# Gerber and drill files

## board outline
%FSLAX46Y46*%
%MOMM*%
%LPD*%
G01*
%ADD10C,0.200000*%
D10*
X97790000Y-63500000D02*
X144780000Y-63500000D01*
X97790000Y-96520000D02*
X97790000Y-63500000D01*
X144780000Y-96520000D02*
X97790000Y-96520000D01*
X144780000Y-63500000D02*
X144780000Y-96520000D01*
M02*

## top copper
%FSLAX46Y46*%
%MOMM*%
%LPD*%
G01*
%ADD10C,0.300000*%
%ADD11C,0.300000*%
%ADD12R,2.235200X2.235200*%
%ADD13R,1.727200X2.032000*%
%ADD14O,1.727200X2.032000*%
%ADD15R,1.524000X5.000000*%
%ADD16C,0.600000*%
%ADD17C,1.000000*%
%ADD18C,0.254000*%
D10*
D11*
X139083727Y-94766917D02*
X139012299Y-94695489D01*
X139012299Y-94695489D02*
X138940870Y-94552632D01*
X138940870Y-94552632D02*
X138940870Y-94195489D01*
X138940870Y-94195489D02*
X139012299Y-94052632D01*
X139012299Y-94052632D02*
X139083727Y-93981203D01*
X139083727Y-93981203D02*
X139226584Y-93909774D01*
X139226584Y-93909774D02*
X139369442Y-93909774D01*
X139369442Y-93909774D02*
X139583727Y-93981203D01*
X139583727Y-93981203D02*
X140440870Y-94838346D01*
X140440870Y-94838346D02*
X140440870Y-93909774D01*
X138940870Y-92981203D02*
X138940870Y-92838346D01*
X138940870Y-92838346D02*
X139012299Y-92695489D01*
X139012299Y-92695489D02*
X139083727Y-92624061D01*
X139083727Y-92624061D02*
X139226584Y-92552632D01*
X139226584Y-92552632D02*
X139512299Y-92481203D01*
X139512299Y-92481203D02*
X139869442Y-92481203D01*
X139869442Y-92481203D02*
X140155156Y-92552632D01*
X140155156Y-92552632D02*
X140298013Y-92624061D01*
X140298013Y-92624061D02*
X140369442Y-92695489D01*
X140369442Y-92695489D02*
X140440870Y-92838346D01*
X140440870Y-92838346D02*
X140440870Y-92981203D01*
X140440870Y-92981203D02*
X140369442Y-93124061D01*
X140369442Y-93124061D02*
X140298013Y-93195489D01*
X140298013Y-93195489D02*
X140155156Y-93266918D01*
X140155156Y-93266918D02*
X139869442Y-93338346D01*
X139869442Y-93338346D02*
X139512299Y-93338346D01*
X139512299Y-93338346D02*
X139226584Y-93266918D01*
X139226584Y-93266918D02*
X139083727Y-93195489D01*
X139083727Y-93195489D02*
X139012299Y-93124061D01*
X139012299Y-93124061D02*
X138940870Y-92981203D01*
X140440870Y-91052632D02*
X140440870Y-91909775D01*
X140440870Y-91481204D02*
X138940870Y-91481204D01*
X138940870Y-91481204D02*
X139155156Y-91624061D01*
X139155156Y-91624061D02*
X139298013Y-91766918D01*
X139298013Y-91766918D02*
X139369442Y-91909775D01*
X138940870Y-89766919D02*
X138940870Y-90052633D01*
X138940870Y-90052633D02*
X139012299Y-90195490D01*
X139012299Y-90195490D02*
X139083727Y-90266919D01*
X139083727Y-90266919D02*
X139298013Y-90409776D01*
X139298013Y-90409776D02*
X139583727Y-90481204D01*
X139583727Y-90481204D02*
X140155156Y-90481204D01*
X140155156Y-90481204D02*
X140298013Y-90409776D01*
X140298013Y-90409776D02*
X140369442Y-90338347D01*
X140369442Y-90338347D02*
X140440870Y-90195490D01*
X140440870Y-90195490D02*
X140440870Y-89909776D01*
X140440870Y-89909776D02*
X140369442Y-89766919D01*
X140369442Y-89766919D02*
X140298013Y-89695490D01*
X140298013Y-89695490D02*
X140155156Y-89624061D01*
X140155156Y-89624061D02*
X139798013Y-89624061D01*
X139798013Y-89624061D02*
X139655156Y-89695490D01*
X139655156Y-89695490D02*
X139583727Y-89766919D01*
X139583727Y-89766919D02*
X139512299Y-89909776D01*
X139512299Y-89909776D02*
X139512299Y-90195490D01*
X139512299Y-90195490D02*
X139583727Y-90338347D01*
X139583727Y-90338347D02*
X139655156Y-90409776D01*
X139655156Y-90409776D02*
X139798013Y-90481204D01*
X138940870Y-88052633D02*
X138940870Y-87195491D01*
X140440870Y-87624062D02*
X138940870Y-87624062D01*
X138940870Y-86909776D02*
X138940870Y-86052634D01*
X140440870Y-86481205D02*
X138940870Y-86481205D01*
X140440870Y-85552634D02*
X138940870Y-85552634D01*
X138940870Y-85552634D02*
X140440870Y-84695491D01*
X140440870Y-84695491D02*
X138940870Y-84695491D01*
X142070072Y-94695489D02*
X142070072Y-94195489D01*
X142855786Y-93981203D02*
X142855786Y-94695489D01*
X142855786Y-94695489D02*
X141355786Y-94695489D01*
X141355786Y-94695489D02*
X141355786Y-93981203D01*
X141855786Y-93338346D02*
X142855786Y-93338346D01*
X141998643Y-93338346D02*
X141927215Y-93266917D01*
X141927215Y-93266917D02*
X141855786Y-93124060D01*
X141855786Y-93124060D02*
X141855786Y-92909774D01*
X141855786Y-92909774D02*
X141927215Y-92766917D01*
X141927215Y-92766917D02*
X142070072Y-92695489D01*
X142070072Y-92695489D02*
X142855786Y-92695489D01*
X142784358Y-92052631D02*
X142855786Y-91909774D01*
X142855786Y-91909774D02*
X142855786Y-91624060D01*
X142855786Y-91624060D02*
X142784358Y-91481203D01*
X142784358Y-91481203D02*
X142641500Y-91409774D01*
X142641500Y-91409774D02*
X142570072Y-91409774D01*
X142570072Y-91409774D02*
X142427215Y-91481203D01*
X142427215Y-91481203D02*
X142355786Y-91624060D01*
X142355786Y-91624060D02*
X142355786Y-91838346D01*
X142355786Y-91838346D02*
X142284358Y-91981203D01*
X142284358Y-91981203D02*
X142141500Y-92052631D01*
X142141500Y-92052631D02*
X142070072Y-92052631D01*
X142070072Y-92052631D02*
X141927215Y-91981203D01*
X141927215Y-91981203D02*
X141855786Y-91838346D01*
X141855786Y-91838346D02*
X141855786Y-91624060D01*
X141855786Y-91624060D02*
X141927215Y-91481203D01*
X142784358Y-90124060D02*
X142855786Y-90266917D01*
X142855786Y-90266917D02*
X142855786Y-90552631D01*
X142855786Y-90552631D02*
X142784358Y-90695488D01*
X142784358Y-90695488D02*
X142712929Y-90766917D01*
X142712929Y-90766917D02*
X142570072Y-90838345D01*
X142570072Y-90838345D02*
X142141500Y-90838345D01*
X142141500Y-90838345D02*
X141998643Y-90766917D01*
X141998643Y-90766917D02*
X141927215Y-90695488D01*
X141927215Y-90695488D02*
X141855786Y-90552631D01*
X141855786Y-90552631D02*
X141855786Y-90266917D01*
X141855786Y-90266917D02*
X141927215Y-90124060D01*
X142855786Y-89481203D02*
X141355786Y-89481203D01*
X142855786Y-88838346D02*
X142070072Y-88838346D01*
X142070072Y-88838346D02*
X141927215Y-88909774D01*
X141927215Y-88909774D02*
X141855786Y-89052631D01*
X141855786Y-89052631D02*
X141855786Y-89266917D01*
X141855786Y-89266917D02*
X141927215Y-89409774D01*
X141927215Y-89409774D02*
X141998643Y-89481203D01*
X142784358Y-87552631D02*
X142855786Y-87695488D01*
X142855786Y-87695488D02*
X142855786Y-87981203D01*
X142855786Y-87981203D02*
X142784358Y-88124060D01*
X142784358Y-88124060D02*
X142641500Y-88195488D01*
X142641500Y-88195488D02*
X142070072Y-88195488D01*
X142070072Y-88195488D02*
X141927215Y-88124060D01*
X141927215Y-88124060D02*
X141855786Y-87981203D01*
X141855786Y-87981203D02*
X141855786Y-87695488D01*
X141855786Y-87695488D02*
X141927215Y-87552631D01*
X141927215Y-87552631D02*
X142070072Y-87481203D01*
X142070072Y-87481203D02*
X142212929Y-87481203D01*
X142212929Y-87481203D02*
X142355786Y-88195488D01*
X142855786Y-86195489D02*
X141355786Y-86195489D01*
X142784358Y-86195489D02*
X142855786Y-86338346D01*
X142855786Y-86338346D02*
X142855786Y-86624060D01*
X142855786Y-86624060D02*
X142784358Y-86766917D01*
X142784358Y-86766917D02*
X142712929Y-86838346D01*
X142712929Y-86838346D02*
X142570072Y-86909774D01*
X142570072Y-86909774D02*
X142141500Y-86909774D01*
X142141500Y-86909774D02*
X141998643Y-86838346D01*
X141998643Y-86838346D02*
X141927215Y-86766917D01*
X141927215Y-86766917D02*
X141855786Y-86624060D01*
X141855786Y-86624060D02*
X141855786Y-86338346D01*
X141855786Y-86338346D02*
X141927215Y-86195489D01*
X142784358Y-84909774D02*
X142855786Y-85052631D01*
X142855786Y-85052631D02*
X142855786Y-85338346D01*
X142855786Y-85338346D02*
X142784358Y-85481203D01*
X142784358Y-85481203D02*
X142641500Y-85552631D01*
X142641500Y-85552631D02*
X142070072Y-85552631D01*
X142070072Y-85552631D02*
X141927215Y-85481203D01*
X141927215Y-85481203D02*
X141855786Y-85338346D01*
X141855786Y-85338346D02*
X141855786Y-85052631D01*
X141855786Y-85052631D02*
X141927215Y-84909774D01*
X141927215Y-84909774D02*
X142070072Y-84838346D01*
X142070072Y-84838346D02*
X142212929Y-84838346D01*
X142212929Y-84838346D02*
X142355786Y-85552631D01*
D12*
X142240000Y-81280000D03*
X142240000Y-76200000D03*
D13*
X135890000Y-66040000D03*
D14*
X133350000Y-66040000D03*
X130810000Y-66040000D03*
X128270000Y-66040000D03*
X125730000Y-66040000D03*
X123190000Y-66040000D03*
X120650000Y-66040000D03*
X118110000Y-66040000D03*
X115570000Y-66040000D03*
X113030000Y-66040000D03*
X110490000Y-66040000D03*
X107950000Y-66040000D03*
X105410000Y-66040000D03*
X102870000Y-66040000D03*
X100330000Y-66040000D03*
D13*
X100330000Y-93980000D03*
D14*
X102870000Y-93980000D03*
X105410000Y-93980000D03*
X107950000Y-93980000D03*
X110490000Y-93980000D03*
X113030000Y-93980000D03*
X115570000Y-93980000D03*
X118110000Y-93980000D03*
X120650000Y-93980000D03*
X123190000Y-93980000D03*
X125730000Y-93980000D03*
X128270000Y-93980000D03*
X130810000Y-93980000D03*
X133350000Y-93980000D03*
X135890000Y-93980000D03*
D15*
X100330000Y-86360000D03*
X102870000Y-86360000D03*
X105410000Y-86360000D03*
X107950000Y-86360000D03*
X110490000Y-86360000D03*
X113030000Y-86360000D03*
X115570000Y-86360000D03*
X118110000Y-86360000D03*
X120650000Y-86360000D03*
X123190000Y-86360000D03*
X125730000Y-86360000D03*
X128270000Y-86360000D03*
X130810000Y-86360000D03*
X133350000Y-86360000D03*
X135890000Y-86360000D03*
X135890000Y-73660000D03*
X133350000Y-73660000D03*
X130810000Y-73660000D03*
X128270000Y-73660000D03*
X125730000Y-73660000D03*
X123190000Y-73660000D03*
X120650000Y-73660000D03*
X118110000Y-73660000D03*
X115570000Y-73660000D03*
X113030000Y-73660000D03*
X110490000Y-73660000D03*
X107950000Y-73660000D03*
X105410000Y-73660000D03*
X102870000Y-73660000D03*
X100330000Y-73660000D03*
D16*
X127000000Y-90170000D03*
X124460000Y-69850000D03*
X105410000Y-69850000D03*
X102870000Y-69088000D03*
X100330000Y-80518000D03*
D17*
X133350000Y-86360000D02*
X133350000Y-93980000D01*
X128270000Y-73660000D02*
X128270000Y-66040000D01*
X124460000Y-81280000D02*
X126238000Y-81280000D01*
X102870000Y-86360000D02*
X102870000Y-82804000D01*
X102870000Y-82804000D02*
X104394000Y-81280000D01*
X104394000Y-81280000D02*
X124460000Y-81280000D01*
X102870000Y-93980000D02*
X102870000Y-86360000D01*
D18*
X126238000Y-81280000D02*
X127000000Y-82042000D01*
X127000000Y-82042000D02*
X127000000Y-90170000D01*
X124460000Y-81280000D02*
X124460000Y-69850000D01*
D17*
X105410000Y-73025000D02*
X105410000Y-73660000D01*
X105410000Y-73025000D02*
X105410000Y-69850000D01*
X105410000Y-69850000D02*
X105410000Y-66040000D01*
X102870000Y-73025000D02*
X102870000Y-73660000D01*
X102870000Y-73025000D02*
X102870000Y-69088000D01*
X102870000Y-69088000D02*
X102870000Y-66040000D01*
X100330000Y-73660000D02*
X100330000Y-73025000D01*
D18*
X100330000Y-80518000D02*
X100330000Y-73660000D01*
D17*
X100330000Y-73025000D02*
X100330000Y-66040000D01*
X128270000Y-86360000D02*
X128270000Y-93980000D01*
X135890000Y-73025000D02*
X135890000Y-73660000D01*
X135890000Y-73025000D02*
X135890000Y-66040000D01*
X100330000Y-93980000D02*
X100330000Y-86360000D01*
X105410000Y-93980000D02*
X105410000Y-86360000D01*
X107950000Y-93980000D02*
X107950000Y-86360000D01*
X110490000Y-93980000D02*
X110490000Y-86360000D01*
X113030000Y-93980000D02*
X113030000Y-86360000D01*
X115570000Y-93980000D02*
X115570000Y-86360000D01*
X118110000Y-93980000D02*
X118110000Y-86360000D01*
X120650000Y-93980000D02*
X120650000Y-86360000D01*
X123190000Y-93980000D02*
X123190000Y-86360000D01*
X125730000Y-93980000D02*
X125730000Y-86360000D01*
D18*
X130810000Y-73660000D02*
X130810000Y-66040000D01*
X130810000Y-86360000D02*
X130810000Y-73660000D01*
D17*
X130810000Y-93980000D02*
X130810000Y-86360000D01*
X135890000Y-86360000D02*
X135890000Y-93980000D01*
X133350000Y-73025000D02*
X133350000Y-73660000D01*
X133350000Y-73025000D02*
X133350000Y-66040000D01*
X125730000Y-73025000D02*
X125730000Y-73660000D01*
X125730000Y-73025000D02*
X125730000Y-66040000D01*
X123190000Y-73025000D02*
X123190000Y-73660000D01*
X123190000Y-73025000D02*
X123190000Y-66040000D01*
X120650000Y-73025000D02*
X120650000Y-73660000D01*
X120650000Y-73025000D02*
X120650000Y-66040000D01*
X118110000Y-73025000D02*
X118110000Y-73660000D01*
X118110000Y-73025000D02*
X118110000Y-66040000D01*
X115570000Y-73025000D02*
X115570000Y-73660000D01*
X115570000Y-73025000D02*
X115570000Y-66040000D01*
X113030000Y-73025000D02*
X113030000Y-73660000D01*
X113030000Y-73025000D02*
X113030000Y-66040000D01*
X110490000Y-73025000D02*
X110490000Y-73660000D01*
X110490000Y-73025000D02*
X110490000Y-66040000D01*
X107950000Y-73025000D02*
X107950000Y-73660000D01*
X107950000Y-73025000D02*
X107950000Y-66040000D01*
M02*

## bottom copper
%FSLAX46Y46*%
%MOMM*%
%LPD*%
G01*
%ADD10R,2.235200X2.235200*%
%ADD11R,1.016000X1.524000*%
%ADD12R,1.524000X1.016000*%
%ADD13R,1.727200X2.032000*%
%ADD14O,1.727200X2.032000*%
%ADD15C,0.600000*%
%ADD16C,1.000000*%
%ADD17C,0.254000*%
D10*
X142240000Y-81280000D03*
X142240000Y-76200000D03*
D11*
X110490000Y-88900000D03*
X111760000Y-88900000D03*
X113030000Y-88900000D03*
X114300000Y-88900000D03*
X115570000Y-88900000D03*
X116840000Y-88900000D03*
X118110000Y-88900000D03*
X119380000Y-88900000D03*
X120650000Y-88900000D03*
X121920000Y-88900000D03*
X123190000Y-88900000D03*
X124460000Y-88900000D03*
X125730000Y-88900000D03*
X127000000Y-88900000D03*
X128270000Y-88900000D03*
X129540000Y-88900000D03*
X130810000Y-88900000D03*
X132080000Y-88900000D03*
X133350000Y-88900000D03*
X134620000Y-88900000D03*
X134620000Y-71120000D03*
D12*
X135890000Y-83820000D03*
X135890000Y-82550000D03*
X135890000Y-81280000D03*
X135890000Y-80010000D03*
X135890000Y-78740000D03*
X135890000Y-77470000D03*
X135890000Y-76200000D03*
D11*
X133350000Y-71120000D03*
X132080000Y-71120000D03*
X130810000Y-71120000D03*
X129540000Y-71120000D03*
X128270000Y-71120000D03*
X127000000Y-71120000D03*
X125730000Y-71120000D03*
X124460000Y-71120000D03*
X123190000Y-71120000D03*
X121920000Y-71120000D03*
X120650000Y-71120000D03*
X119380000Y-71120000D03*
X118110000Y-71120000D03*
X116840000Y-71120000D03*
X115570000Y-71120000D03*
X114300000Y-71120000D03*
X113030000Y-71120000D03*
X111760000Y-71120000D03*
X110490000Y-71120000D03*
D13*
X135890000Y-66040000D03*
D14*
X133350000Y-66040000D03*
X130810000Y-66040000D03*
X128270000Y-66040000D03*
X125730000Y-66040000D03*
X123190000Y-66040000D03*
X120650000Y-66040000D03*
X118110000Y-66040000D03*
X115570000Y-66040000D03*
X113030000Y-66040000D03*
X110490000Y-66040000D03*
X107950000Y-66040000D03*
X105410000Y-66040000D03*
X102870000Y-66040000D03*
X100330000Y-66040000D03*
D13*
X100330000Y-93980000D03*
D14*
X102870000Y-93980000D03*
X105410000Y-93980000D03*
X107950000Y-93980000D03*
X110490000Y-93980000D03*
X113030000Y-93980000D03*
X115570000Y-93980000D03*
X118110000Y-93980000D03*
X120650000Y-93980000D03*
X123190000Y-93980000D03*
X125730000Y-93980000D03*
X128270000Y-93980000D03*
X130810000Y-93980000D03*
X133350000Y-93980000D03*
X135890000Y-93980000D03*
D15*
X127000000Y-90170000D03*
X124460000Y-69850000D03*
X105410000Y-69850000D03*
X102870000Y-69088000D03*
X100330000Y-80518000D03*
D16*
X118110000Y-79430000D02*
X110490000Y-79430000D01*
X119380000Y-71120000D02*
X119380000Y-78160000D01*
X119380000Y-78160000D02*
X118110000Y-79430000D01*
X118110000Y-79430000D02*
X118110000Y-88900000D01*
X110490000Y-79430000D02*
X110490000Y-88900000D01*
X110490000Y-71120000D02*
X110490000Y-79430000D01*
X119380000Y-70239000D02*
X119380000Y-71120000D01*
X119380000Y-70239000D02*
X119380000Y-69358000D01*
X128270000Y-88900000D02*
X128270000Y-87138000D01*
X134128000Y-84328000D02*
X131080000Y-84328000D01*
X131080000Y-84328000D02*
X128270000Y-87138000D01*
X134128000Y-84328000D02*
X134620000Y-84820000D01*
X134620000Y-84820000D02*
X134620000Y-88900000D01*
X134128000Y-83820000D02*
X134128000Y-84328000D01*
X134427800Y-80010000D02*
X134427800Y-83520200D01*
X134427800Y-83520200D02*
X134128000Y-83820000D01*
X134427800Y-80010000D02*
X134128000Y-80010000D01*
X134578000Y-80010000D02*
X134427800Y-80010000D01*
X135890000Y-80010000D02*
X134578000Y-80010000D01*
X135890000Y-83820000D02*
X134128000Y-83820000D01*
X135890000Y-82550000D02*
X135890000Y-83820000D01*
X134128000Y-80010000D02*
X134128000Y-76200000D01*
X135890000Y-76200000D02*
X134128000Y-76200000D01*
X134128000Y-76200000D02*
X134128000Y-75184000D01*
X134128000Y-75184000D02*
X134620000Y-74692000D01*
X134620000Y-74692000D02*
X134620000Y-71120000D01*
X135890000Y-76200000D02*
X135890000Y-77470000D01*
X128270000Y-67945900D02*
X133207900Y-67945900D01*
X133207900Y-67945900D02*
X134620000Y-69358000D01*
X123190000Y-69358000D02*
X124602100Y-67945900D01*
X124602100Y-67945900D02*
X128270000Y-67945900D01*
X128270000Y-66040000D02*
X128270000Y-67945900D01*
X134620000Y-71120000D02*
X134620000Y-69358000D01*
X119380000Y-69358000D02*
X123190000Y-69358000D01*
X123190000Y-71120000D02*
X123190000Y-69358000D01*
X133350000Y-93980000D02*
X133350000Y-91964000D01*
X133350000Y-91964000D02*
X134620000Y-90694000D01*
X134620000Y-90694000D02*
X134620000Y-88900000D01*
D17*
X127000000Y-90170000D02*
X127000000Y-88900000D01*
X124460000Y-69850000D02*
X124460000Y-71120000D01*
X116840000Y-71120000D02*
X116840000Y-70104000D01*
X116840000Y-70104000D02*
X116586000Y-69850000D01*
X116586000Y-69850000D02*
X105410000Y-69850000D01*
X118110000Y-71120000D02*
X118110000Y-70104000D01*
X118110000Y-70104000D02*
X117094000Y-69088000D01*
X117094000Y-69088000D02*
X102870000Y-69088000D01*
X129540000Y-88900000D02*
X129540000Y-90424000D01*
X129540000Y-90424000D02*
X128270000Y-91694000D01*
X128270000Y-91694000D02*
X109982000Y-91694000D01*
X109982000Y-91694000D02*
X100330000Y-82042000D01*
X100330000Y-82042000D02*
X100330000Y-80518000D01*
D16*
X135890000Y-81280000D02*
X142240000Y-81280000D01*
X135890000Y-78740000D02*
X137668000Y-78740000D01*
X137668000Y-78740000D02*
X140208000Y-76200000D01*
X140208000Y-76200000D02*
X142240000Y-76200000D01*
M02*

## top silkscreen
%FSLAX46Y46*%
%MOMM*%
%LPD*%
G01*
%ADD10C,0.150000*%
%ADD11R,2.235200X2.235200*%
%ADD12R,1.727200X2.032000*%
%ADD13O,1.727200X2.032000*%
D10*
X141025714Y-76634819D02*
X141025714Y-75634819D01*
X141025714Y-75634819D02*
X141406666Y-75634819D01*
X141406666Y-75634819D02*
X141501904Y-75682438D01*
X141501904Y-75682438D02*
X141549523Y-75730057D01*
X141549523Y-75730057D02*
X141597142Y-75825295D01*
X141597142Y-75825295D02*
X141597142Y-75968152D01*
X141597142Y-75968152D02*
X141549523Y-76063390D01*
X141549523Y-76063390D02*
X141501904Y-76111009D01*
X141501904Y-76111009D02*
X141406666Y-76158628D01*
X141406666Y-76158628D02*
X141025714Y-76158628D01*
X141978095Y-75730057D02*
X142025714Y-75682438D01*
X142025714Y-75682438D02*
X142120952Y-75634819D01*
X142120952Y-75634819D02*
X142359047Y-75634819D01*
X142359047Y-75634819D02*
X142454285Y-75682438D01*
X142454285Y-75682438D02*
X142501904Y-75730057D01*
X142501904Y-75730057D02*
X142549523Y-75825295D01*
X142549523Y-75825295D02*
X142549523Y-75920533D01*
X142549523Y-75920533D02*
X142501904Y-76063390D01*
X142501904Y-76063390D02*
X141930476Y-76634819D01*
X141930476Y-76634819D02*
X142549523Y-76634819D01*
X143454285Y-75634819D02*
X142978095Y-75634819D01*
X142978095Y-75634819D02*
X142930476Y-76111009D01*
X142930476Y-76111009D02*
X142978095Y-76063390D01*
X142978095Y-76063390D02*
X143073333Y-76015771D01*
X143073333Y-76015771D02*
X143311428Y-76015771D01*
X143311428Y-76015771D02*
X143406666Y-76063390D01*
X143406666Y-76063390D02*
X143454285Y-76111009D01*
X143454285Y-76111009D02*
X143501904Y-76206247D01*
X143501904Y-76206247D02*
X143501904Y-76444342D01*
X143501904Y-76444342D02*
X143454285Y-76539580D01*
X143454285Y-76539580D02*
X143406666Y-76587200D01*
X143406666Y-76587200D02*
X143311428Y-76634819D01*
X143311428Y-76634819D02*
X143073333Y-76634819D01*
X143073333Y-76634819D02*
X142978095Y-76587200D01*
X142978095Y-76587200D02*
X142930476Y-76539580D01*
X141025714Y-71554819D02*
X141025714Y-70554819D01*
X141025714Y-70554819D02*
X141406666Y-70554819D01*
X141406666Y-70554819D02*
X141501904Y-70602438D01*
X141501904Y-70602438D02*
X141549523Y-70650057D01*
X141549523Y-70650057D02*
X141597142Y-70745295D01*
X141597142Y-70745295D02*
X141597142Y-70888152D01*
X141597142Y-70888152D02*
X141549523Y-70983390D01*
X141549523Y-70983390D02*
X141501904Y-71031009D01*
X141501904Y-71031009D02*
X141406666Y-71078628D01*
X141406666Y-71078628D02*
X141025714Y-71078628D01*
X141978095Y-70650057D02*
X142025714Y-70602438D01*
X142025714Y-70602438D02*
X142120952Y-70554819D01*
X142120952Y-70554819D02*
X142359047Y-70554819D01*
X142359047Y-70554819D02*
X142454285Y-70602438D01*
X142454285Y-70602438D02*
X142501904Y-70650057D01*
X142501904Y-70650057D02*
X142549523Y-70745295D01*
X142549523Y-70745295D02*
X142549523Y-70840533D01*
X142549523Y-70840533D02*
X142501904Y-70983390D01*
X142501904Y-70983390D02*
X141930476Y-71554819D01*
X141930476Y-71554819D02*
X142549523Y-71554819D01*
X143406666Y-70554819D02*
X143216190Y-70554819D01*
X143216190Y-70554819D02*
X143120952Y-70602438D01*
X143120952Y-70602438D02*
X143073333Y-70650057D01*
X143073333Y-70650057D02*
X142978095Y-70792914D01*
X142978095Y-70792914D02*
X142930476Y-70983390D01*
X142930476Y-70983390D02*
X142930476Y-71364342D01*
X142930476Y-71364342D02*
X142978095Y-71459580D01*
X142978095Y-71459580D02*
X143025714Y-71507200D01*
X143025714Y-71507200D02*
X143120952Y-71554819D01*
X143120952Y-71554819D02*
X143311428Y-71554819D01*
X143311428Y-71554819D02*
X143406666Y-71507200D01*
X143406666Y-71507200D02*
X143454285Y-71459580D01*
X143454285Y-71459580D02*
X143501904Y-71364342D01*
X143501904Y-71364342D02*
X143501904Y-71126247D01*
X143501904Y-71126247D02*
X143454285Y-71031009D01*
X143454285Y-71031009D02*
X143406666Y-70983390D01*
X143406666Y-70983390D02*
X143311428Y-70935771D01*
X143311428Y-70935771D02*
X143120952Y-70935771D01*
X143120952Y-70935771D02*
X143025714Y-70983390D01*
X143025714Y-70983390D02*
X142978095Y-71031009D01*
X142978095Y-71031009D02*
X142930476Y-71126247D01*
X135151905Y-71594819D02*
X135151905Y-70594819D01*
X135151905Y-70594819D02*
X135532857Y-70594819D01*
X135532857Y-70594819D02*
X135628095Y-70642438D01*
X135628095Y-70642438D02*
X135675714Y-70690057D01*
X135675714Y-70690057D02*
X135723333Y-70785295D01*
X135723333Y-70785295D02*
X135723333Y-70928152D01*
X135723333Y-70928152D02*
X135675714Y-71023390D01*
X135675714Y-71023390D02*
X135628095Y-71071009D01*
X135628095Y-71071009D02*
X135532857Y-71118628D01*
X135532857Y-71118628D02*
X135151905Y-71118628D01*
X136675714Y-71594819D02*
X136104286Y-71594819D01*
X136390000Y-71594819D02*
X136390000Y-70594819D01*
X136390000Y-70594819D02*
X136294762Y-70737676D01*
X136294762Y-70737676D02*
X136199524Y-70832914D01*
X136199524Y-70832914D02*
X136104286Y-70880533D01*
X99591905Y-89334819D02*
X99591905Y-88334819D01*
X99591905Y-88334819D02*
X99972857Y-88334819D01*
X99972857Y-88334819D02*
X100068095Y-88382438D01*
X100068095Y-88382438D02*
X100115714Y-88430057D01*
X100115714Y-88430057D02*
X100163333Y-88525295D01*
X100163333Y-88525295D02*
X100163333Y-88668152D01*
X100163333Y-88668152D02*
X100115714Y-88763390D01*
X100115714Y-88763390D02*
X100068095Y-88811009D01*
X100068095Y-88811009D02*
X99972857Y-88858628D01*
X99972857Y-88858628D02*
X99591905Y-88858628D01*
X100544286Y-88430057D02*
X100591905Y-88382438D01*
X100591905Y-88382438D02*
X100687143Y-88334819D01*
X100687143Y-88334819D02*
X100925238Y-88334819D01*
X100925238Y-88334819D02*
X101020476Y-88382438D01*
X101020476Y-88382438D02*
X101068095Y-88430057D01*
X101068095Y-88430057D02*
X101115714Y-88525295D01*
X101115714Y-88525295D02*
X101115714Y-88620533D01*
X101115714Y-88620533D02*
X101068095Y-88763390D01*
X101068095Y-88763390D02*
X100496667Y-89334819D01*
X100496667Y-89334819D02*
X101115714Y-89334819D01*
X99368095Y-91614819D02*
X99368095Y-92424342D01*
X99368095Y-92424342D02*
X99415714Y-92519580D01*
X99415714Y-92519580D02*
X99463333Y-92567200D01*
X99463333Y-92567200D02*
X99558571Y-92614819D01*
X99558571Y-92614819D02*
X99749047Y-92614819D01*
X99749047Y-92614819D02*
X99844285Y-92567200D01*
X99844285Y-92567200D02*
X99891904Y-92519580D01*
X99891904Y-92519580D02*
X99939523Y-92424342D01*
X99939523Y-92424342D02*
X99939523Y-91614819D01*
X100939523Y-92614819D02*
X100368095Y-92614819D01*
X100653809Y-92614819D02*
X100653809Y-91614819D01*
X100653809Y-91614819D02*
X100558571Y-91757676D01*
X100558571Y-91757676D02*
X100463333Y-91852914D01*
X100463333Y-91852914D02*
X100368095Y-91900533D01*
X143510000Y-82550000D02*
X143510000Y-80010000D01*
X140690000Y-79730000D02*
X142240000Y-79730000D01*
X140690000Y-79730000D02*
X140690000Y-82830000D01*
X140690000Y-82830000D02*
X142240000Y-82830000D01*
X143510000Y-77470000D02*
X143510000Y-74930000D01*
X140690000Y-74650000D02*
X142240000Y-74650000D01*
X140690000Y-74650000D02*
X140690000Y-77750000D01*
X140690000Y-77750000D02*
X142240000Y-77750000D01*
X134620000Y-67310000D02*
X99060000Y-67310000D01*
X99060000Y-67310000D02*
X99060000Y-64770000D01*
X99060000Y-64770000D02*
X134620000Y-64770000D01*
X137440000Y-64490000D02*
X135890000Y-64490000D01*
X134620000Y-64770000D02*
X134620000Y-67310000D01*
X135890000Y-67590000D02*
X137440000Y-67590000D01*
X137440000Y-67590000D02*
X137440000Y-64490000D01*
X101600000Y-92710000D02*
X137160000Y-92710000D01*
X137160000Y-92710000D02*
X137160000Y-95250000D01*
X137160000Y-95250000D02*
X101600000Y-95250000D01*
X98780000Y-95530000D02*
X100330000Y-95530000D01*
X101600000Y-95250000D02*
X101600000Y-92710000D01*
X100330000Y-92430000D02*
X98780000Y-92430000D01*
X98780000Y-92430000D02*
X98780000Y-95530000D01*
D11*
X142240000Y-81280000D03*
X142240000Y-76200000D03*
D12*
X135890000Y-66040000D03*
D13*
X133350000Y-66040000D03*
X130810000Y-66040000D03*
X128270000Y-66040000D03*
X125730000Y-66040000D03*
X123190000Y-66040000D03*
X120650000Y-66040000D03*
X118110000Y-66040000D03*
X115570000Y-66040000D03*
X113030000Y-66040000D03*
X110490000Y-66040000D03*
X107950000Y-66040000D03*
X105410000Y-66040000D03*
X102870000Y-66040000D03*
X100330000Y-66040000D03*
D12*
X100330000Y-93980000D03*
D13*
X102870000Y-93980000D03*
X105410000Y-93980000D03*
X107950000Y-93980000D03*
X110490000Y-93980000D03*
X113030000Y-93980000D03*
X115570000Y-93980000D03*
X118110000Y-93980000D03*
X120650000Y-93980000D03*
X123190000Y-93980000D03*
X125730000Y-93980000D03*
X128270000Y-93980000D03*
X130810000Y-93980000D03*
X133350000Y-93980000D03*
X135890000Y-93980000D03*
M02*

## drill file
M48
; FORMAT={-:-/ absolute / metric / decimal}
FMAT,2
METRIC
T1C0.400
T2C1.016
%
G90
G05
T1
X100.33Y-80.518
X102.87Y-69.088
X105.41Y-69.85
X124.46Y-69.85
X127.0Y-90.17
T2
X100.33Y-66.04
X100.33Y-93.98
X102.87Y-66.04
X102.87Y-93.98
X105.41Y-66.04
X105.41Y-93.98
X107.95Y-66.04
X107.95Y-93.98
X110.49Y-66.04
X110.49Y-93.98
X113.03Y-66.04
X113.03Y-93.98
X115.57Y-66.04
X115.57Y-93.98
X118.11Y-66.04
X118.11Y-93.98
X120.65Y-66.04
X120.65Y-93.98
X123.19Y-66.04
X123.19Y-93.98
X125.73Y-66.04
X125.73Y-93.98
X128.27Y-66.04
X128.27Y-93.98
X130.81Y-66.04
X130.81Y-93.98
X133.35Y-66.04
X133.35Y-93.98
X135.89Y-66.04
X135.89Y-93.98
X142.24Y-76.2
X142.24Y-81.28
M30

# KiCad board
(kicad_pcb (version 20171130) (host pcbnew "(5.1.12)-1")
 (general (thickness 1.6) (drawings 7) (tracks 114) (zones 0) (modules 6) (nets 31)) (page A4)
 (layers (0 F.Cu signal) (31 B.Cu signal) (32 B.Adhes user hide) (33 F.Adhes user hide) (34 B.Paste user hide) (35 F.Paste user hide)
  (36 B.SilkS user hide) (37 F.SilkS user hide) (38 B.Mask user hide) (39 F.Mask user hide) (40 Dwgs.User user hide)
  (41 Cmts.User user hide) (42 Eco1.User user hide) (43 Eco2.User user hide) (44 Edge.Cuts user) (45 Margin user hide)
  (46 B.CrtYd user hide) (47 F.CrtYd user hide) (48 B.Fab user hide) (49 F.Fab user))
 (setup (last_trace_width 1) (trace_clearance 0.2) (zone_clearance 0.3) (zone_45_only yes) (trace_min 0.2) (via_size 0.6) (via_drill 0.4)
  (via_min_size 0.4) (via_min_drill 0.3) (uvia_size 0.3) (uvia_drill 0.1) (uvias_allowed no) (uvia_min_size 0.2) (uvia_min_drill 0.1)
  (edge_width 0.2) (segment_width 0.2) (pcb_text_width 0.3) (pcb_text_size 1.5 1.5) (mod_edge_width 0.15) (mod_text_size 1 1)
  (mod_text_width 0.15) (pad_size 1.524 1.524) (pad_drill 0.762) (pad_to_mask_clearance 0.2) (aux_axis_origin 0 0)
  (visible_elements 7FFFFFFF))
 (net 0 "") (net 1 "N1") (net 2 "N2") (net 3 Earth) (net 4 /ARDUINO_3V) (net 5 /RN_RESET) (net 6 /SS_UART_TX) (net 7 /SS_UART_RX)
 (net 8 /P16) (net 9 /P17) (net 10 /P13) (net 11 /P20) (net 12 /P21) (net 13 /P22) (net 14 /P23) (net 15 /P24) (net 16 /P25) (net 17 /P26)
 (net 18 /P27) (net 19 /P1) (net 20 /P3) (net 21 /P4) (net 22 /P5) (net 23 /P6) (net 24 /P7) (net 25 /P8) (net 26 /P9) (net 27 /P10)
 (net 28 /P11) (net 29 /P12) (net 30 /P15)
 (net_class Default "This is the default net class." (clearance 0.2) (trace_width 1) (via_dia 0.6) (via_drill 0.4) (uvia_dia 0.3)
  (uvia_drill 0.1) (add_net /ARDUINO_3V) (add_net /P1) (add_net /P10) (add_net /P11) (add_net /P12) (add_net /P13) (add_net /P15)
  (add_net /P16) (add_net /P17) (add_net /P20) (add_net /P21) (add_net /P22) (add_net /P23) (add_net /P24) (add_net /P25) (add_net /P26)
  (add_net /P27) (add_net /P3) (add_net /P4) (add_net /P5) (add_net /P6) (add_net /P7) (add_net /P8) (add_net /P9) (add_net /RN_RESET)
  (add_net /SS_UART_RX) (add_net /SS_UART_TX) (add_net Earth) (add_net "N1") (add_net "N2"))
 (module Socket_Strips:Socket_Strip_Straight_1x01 (layer F.Cu) (at 142.24 81.28)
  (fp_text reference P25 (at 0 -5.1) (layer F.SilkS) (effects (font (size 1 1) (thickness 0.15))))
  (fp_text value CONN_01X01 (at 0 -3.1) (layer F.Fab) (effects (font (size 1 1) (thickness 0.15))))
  (fp_line (start 1.27 1.27) (end 1.27 -1.27) (layer F.SilkS) (width 0.15))
  (fp_line (start -1.55 -1.55) (end 0 -1.55) (layer F.SilkS) (width 0.15))
  (fp_line (start -1.55 -1.55) (end -1.55 1.55) (layer F.SilkS) (width 0.15))
  (fp_line (start -1.55 1.55) (end 0 1.55) (layer F.SilkS) (width 0.15))
  (pad 1 thru_hole rect (at 0 0) (size 2.2352 2.2352) (drill 1.016) (layers *.Cu *.Mask F.SilkS) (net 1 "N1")))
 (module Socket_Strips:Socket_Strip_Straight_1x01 (layer F.Cu) (at 142.24 76.2)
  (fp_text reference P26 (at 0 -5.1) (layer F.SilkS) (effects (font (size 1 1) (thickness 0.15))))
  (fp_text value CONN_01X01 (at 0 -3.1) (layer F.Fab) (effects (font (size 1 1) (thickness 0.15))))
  (fp_line (start 1.27 1.27) (end 1.27 -1.27) (layer F.SilkS) (width 0.15))
  (fp_line (start -1.55 -1.55) (end 0 -1.55) (layer F.SilkS) (width 0.15))
  (fp_line (start -1.55 -1.55) (end -1.55 1.55) (layer F.SilkS) (width 0.15))
  (fp_line (start -1.55 1.55) (end 0 1.55) (layer F.SilkS) (width 0.15))
  (pad 1 thru_hole rect (at 0 0) (size 2.2352 2.2352) (drill 1.016) (layers *.Cu *.Mask F.SilkS) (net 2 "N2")))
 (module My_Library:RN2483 (layer B.Cu) (at 109.22 88.9 90)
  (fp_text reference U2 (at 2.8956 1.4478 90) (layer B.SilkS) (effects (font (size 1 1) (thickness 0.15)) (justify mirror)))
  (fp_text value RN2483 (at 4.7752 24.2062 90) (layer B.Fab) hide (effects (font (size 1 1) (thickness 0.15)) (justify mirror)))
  (pad 47 smd rect (at 0 1.27 90) (size 1.524 1.016) (layers B.Cu B.Paste B.Mask) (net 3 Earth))
  (pad 46 smd rect (at 0 2.54 90) (size 1.524 1.016) (layers B.Cu B.Paste B.Mask))
  (pad 45 smd rect (at 0 3.81 90) (size 1.524 1.016) (layers B.Cu B.Paste B.Mask))
  (pad 44 smd rect (at 0 5.08 90) (size 1.524 1.016) (layers B.Cu B.Paste B.Mask))
  (pad 43 smd rect (at 0 6.35 90) (size 1.524 1.016) (layers B.Cu B.Paste B.Mask))
  (pad 42 smd rect (at 0 7.62 90) (size 1.524 1.016) (layers B.Cu B.Paste B.Mask))
  (pad 41 smd rect (at 0 8.89 90) (size 1.524 1.016) (layers B.Cu B.Paste B.Mask) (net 3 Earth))
  (pad 40 smd rect (at 0 10.16 90) (size 1.524 1.016) (layers B.Cu B.Paste B.Mask))
  (pad 39 smd rect (at 0 11.43 90) (size 1.524 1.016) (layers B.Cu B.Paste B.Mask))
  (pad 38 smd rect (at 0 12.7 90) (size 1.524 1.016) (layers B.Cu B.Paste B.Mask))
  (pad 37 smd rect (at 0 13.97 90) (size 1.524 1.016) (layers B.Cu B.Paste B.Mask))
  (pad 36 smd rect (at 0 15.24 90) (size 1.524 1.016) (layers B.Cu B.Paste B.Mask))
  (pad 35 smd rect (at 0 16.51 90) (size 1.524 1.016) (layers B.Cu B.Paste B.Mask))
  (pad 34 smd rect (at 0 17.78 90) (size 1.524 1.016) (layers B.Cu B.Paste B.Mask) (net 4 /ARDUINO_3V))
  (pad 33 smd rect (at 0 19.05 90) (size 1.524 1.016) (layers B.Cu B.Paste B.Mask) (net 3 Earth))
  (pad 32 smd rect (at 0 20.32 90) (size 1.524 1.016) (layers B.Cu B.Paste B.Mask) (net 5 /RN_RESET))
  (pad 31 smd rect (at 0 21.59 90) (size 1.524 1.016) (layers B.Cu B.Paste B.Mask))
  (pad 30 smd rect (at 0 22.86 90) (size 1.524 1.016) (layers B.Cu B.Paste B.Mask))
  (pad 29 smd rect (at 0 24.13 90) (size 1.524 1.016) (layers B.Cu B.Paste B.Mask))
  (pad 28 smd rect (at 0 25.4 90) (size 1.524 1.016) (layers B.Cu B.Paste B.Mask) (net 3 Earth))
  (pad 20 smd rect (at 17.78 25.4 90) (size 1.524 1.016) (layers B.Cu B.Paste B.Mask) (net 3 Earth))
  (pad 27 smd rect (at 5.08 26.67 90) (size 1.016 1.524) (layers B.Cu B.Paste B.Mask) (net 3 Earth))
  (pad 26 smd rect (at 6.35 26.67 90) (size 1.016 1.524) (layers B.Cu B.Paste B.Mask) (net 3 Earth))
  (pad 25 smd rect (at 7.62 26.67 90) (size 1.016 1.524) (layers B.Cu B.Paste B.Mask) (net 1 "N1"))
  (pad 24 smd rect (at 8.89 26.67 90) (size 1.016 1.524) (layers B.Cu B.Paste B.Mask) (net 3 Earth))
  (pad 23 smd rect (at 10.16 26.67 90) (size 1.016 1.524) (layers B.Cu B.Paste B.Mask) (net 2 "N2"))
  (pad 22 smd rect (at 11.43 26.67 90) (size 1.016 1.524) (layers B.Cu B.Paste B.Mask) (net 3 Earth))
  (pad 21 smd rect (at 12.7 26.67 90) (size 1.016 1.524) (layers B.Cu B.Paste B.Mask) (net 3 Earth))
  (pad 19 smd rect (at 17.78 24.13 90) (size 1.524 1.016) (layers B.Cu B.Paste B.Mask))
  (pad 18 smd rect (at 17.78 22.86 90) (size 1.524 1.016) (layers B.Cu B.Paste B.Mask))
  (pad 17 smd rect (at 17.78 21.59 90) (size 1.524 1.016) (layers B.Cu B.Paste B.Mask))
  (pad 16 smd rect (at 17.78 20.32 90) (size 1.524 1.016) (layers B.Cu B.Paste B.Mask))
  (pad 15 smd rect (at 17.78 19.05 90) (size 1.524 1.016) (layers B.Cu B.Paste B.Mask))
  (pad 14 smd rect (at 17.78 17.78 90) (size 1.524 1.016) (layers B.Cu B.Paste B.Mask))
  (pad 13 smd rect (at 17.78 16.51 90) (size 1.524 1.016) (layers B.Cu B.Paste B.Mask))
  (pad 12 smd rect (at 17.78 15.24 90) (size 1.524 1.016) (layers B.Cu B.Paste B.Mask) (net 4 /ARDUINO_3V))
  (pad 11 smd rect (at 17.78 13.97 90) (size 1.524 1.016) (layers B.Cu B.Paste B.Mask) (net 3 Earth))
  (pad 10 smd rect (at 17.78 12.7 90) (size 1.524 1.016) (layers B.Cu B.Paste B.Mask))
  (pad 9 smd rect (at 17.78 11.43 90) (size 1.524 1.016) (layers B.Cu B.Paste B.Mask))
  (pad 8 smd rect (at 17.78 10.16 90) (size 1.524 1.016) (layers B.Cu B.Paste B.Mask) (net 3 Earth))
  (pad 7 smd rect (at 17.78 8.89 90) (size 1.524 1.016) (layers B.Cu B.Paste B.Mask) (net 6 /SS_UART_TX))
  (pad 6 smd rect (at 17.78 7.62 90) (size 1.524 1.016) (layers B.Cu B.Paste B.Mask) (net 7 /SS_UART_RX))
  (pad 5 smd rect (at 17.78 6.35 90) (size 1.524 1.016) (layers B.Cu B.Paste B.Mask))
  (pad 4 smd rect (at 17.78 5.08 90) (size 1.524 1.016) (layers B.Cu B.Paste B.Mask))
  (pad 3 smd rect (at 17.78 3.81 90) (size 1.524 1.016) (layers B.Cu B.Paste B.Mask))
  (pad 2 smd rect (at 17.78 2.54 90) (size 1.524 1.016) (layers B.Cu B.Paste B.Mask))
  (pad 1 smd rect (at 17.78 1.27 90) (size 1.524 1.016) (layers B.Cu B.Paste B.Mask) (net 3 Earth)))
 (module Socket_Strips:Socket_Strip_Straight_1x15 (layer F.Cu) (at 135.89 66.04 180)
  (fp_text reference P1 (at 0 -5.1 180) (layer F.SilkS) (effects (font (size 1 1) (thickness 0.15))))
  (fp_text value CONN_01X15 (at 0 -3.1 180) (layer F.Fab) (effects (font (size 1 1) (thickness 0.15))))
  (fp_line (start 1.27 -1.27) (end 36.83 -1.27) (layer F.SilkS) (width 0.15))
  (fp_line (start 36.83 -1.27) (end 36.83 1.27) (layer F.SilkS) (width 0.15))
  (fp_line (start 36.83 1.27) (end 1.27 1.27) (layer F.SilkS) (width 0.15))
  (fp_line (start -1.55 1.55) (end 0 1.55) (layer F.SilkS) (width 0.15))
  (fp_line (start 1.27 1.27) (end 1.27 -1.27) (layer F.SilkS) (width 0.15))
  (fp_line (start 0 -1.55) (end -1.55 -1.55) (layer F.SilkS) (width 0.15))
  (fp_line (start -1.55 -1.55) (end -1.55 1.55) (layer F.SilkS) (width 0.15))
  (pad 1 thru_hole rect (at 0 0 180) (size 1.7272 2.032) (drill 1.016) (layers *.Cu *.Mask F.SilkS) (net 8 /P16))
  (pad 2 thru_hole oval (at 2.54 0 180) (size 1.7272 2.032) (drill 1.016) (layers *.Cu *.Mask F.SilkS) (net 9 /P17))
  (pad 3 thru_hole oval (at 5.08 0 180) (size 1.7272 2.032) (drill 1.016) (layers *.Cu *.Mask F.SilkS) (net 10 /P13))
  (pad 4 thru_hole oval (at 7.62 0 180) (size 1.7272 2.032) (drill 1.016) (layers *.Cu *.Mask F.SilkS) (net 3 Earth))
  (pad 5 thru_hole oval (at 10.16 0 180) (size 1.7272 2.032) (drill 1.016) (layers *.Cu *.Mask F.SilkS) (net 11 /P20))
  (pad 6 thru_hole oval (at 12.7 0 180) (size 1.7272 2.032) (drill 1.016) (layers *.Cu *.Mask F.SilkS) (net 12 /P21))
  (pad 7 thru_hole oval (at 15.24 0 180) (size 1.7272 2.032) (drill 1.016) (layers *.Cu *.Mask F.SilkS) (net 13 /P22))
  (pad 8 thru_hole oval (at 17.78 0 180) (size 1.7272 2.032) (drill 1.016) (layers *.Cu *.Mask F.SilkS) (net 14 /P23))
  (pad 9 thru_hole oval (at 20.32 0 180) (size 1.7272 2.032) (drill 1.016) (layers *.Cu *.Mask F.SilkS) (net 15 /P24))
  (pad 10 thru_hole oval (at 22.86 0 180) (size 1.7272 2.032) (drill 1.016) (layers *.Cu *.Mask F.SilkS) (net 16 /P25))
  (pad 11 thru_hole oval (at 25.4 0 180) (size 1.7272 2.032) (drill 1.016) (layers *.Cu *.Mask F.SilkS) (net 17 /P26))
  (pad 12 thru_hole oval (at 27.94 0 180) (size 1.7272 2.032) (drill 1.016) (layers *.Cu *.Mask F.SilkS) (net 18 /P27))
  (pad 13 thru_hole oval (at 30.48 0 180) (size 1.7272 2.032) (drill 1.016) (layers *.Cu *.Mask F.SilkS) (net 7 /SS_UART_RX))
  (pad 14 thru_hole oval (at 33.02 0 180) (size 1.7272 2.032) (drill 1.016) (layers *.Cu *.Mask F.SilkS) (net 6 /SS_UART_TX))
  (pad 15 thru_hole oval (at 35.56 0 180) (size 1.7272 2.032) (drill 1.016) (layers *.Cu *.Mask F.SilkS) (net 5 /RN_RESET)))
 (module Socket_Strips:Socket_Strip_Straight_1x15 (layer F.Cu) (at 100.33 93.98)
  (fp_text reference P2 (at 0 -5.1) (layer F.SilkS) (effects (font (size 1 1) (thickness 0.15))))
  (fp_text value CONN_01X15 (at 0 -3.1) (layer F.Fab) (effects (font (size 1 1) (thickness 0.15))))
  (fp_line (start 1.27 -1.27) (end 36.83 -1.27) (layer F.SilkS) (width 0.15))
  (fp_line (start 36.83 -1.27) (end 36.83 1.27) (layer F.SilkS) (width 0.15))
  (fp_line (start 36.83 1.27) (end 1.27 1.27) (layer F.SilkS) (width 0.15))
  (fp_line (start -1.55 1.55) (end 0 1.55) (layer F.SilkS) (width 0.15))
  (fp_line (start 1.27 1.27) (end 1.27 -1.27) (layer F.SilkS) (width 0.15))
  (fp_line (start 0 -1.55) (end -1.55 -1.55) (layer F.SilkS) (width 0.15))
  (fp_line (start -1.55 -1.55) (end -1.55 1.55) (layer F.SilkS) (width 0.15))
  (pad 1 thru_hole rect (at 0 0) (size 1.7272 2.032) (drill 1.016) (layers *.Cu *.Mask F.SilkS) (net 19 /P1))
  (pad 2 thru_hole oval (at 2.54 0) (size 1.7272 2.032) (drill 1.016) (layers *.Cu *.Mask F.SilkS) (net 4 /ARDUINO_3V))
  (pad 3 thru_hole oval (at 5.08 0) (size 1.7272 2.032) (drill 1.016) (layers *.Cu *.Mask F.SilkS) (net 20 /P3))
  (pad 4 thru_hole oval (at 7.62 0) (size 1.7272 2.032) (drill 1.016) (layers *.Cu *.Mask F.SilkS) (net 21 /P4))
  (pad 5 thru_hole oval (at 10.16 0) (size 1.7272 2.032) (drill 1.016) (layers *.Cu *.Mask F.SilkS) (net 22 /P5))
  (pad 6 thru_hole oval (at 12.7 0) (size 1.7272 2.032) (drill 1.016) (layers *.Cu *.Mask F.SilkS) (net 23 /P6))
  (pad 7 thru_hole oval (at 15.24 0) (size 1.7272 2.032) (drill 1.016) (layers *.Cu *.Mask F.SilkS) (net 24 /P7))
  (pad 8 thru_hole oval (at 17.78 0) (size 1.7272 2.032) (drill 1.016) (layers *.Cu *.Mask F.SilkS) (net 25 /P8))
  (pad 9 thru_hole oval (at 20.32 0) (size 1.7272 2.032) (drill 1.016) (layers *.Cu *.Mask F.SilkS) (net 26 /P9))
  (pad 10 thru_hole oval (at 22.86 0) (size 1.7272 2.032) (drill 1.016) (layers *.Cu *.Mask F.SilkS) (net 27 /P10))
  (pad 11 thru_hole oval (at 25.4 0) (size 1.7272 2.032) (drill 1.016) (layers *.Cu *.Mask F.SilkS) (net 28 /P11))
  (pad 12 thru_hole oval (at 27.94 0) (size 1.7272 2.032) (drill 1.016) (layers *.Cu *.Mask F.SilkS) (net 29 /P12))
  (pad 13 thru_hole oval (at 30.48 0) (size 1.7272 2.032) (drill 1.016) (layers *.Cu *.Mask F.SilkS) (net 10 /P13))
  (pad 14 thru_hole oval (at 33.02 0) (size 1.7272 2.032) (drill 1.016) (layers *.Cu *.Mask F.SilkS) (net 3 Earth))
  (pad 15 thru_hole oval (at 35.56 0) (size 1.7272 2.032) (drill 1.016) (layers *.Cu *.Mask F.SilkS) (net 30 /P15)))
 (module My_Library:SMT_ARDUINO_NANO (layer F.Cu) (at 100.33 86.36)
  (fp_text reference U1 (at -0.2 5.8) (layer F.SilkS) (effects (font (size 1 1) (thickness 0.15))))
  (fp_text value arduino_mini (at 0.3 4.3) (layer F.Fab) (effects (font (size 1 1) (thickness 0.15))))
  (pad 1 smd rect (at 0 0) (size 1.524 5) (layers F.Cu F.Paste F.Mask) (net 19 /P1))
  (pad 2 smd rect (at 2.54 0) (size 1.524 5) (layers F.Cu F.Paste F.Mask) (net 4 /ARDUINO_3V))
  (pad 3 smd rect (at 5.08 0) (size 1.524 5) (layers F.Cu F.Paste F.Mask) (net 20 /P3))
  (pad 4 smd rect (at 7.62 0) (size 1.524 5) (layers F.Cu F.Paste F.Mask) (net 21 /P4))
  (pad 5 smd rect (at 10.16 0) (size 1.524 5) (layers F.Cu F.Paste F.Mask) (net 22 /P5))
  (pad 6 smd rect (at 12.7 0) (size 1.524 5) (layers F.Cu F.Paste F.Mask) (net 23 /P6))
  (pad 7 smd rect (at 15.24 0) (size 1.524 5) (layers F.Cu F.Paste F.Mask) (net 24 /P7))
  (pad 8 smd rect (at 17.78 0) (size 1.524 5) (layers F.Cu F.Paste F.Mask) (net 25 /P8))
  (pad 9 smd rect (at 20.32 0) (size 1.524 5) (layers F.Cu F.Paste F.Mask) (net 26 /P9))
  (pad 10 smd rect (at 22.86 0) (size 1.524 5) (layers F.Cu F.Paste F.Mask) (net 27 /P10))
  (pad 11 smd rect (at 25.4 0) (size 1.524 5) (layers F.Cu F.Paste F.Mask) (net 28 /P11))
  (pad 12 smd rect (at 27.94 0) (size 1.524 5) (layers F.Cu F.Paste F.Mask) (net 29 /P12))
  (pad 13 smd rect (at 30.48 0) (size 1.524 5) (layers F.Cu F.Paste F.Mask) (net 10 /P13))
  (pad 14 smd rect (at 33.02 0) (size 1.524 5) (layers F.Cu F.Paste F.Mask) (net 3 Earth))
  (pad 15 smd rect (at 35.56 0) (size 1.524 5) (layers F.Cu F.Paste F.Mask) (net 30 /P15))
  (pad 16 smd rect (at 35.56 -12.7) (size 1.524 5) (layers F.Cu F.Paste F.Mask) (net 8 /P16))
  (pad 17 smd rect (at 33.02 -12.7) (size 1.524 5) (layers F.Cu F.Paste F.Mask) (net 9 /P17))
  (pad 18 smd rect (at 30.48 -12.7) (size 1.524 5) (layers F.Cu F.Paste F.Mask) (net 10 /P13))
  (pad 19 smd rect (at 27.94 -12.7) (size 1.524 5) (layers F.Cu F.Paste F.Mask) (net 3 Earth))
  (pad 20 smd rect (at 25.4 -12.7) (size 1.524 5) (layers F.Cu F.Paste F.Mask) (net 11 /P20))
  (pad 21 smd rect (at 22.86 -12.7) (size 1.524 5) (layers F.Cu F.Paste F.Mask) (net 12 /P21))
  (pad 22 smd rect (at 20.32 -12.7) (size 1.524 5) (layers F.Cu F.Paste F.Mask) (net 13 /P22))
  (pad 23 smd rect (at 17.78 -12.7) (size 1.524 5) (layers F.Cu F.Paste F.Mask) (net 14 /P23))
  (pad 24 smd rect (at 15.24 -12.7) (size 1.524 5) (layers F.Cu F.Paste F.Mask) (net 15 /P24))
  (pad 25 smd rect (at 12.7 -12.7) (size 1.524 5) (layers F.Cu F.Paste F.Mask) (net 16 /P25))
  (pad 26 smd rect (at 10.16 -12.7) (size 1.524 5) (layers F.Cu F.Paste F.Mask) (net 17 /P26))
  (pad 27 smd rect (at 7.62 -12.7) (size 1.524 5) (layers F.Cu F.Paste F.Mask) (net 18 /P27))
  (pad 28 smd rect (at 5.08 -12.7) (size 1.524 5) (layers F.Cu F.Paste F.Mask) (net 7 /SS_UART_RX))
  (pad 29 smd rect (at 2.54 -12.7) (size 1.524 5) (layers F.Cu F.Paste F.Mask) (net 6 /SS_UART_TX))
  (pad 30 smd rect (at 0 -12.7) (size 1.524 5) (layers F.Cu F.Paste F.Mask) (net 5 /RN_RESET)))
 (gr_line (start 97.79 63.5) (end 144.78 63.5) (angle 90) (layer Edge.Cuts) (width 0.2))
 (gr_line (start 97.79 96.52) (end 97.79 63.5) (angle 90) (layer Edge.Cuts) (width 0.2))
 (gr_line (start 144.78 96.52) (end 97.79 96.52) (angle 90) (layer Edge.Cuts) (width 0.2))
 (gr_line (start 144.78 63.5) (end 144.78 96.52) (angle 90) (layer Edge.Cuts) (width 0.2))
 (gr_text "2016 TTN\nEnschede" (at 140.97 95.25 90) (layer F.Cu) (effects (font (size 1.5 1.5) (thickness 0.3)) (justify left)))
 (segment (start 118.11 79.43) (end 110.49 79.43) (width 1) (layer B.Cu) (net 3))
 (segment (start 119.38 71.12) (end 119.38 78.16) (width 1) (layer B.Cu) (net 3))
 (segment (start 119.38 78.16) (end 118.11 79.43) (width 1) (layer B.Cu) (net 3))
 (segment (start 118.11 79.43) (end 118.11 88.9) (width 1) (layer B.Cu) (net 3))
 (segment (start 110.49 79.43) (end 110.49 88.9) (width 1) (layer B.Cu) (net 3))
 (segment (start 110.49 71.12) (end 110.49 79.43) (width 1) (layer B.Cu) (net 3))
 (segment (start 119.38 70.239) (end 119.38 71.12) (width 1) (layer B.Cu) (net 3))
 (segment (start 119.38 70.239) (end 119.38 69.358) (width 1) (layer B.Cu) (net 3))
 (segment (start 128.27 88.9) (end 128.27 87.138) (width 1) (layer B.Cu) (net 3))
 (segment (start 134.128 84.328) (end 131.08 84.328) (width 1) (layer B.Cu) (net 3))
 (segment (start 131.08 84.328) (end 128.27 87.138) (width 1) (layer B.Cu) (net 3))
 (segment (start 134.128 84.328) (end 134.62 84.82) (width 1) (layer B.Cu) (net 3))
 (segment (start 134.62 84.82) (end 134.62 88.9) (width 1) (layer B.Cu) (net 3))
 (segment (start 134.128 83.82) (end 134.128 84.328) (width 1) (layer B.Cu) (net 3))
 (segment (start 134.4278 80.01) (end 134.4278 83.5202) (width 1) (layer B.Cu) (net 3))
 (segment (start 134.4278 83.5202) (end 134.128 83.82) (width 1) (layer B.Cu) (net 3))
 (segment (start 134.4278 80.01) (end 134.128 80.01) (width 1) (layer B.Cu) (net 3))
 (segment (start 134.578 80.01) (end 134.4278 80.01) (width 1) (layer B.Cu) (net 3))
 (segment (start 135.89 80.01) (end 134.578 80.01) (width 1) (layer B.Cu) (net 3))
 (segment (start 135.89 83.82) (end 134.128 83.82) (width 1) (layer B.Cu) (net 3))
 (segment (start 135.89 82.55) (end 135.89 83.82) (width 1) (layer B.Cu) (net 3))
 (segment (start 134.128 80.01) (end 134.128 76.2) (width 1) (layer B.Cu) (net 3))
 (segment (start 135.89 76.2) (end 134.128 76.2) (width 1) (layer B.Cu) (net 3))
 (segment (start 134.128 76.2) (end 134.128 75.184) (width 1) (layer B.Cu) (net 3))
 (segment (start 134.128 75.184) (end 134.62 74.692) (width 1) (layer B.Cu) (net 3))
 (segment (start 134.62 74.692) (end 134.62 71.12) (width 1) (layer B.Cu) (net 3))
 (segment (start 135.89 76.2) (end 135.89 77.47) (width 1) (layer B.Cu) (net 3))
 (segment (start 128.27 67.9459) (end 133.2079 67.9459) (width 1) (layer B.Cu) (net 3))
 (segment (start 133.2079 67.9459) (end 134.62 69.358) (width 1) (layer B.Cu) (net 3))
 (segment (start 123.19 69.358) (end 124.6021 67.9459) (width 1) (layer B.Cu) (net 3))
 (segment (start 124.6021 67.9459) (end 128.27 67.9459) (width 1) (layer B.Cu) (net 3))
 (segment (start 128.27 66.04) (end 128.27 67.9459) (width 1) (layer B.Cu) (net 3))
 (segment (start 134.62 71.12) (end 134.62 69.358) (width 1) (layer B.Cu) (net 3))
 (segment (start 119.38 69.358) (end 123.19 69.358) (width 1) (layer B.Cu) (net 3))
 (segment (start 123.19 71.12) (end 123.19 69.358) (width 1) (layer B.Cu) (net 3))
 (segment (start 133.35 93.98) (end 133.35 91.964) (width 1) (layer B.Cu) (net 3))
 (segment (start 133.35 91.964) (end 134.62 90.694) (width 1) (layer B.Cu) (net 3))
 (segment (start 134.62 90.694) (end 134.62 88.9) (width 1) (layer B.Cu) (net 3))
 (segment (start 133.35 86.36) (end 133.35 93.98) (width 1) (layer F.Cu) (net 3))
 (segment (start 128.27 73.66) (end 128.27 66.04) (width 1) (layer F.Cu) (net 3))
 (segment (start 124.46 81.28) (end 126.238 81.28) (width 1) (layer F.Cu) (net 4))
 (segment (start 102.87 86.36) (end 102.87 82.804) (width 1) (layer F.Cu) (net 4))
 (segment (start 102.87 82.804) (end 104.394 81.28) (width 1) (layer F.Cu) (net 4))
 (segment (start 104.394 81.28) (end 124.46 81.28) (width 1) (layer F.Cu) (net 4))
 (segment (start 102.87 93.98) (end 102.87 86.36) (width 1) (layer F.Cu) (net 4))
 (segment (start 126.238 81.28) (end 127 82.042) (width 0.254) (layer F.Cu) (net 4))
 (segment (start 127 82.042) (end 127 90.17) (width 0.254) (layer F.Cu) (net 4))
 (segment (start 127 90.17) (end 127 88.9) (width 0.254) (layer B.Cu) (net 4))
 (segment (start 124.46 69.85) (end 124.46 71.12) (width 0.254) (layer B.Cu) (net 4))
 (segment (start 124.46 81.28) (end 124.46 69.85) (width 0.254) (layer F.Cu) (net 4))
 (via (at 127 90.17) (size 0.6) (layers F.Cu B.Cu) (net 4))
 (via (at 124.46 69.85) (size 0.6) (layers F.Cu B.Cu) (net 4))
 (segment (start 105.41 73.025) (end 105.41 73.66) (width 1) (layer F.Cu) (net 7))
 (segment (start 105.41 73.025) (end 105.41 69.85) (width 1) (layer F.Cu) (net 7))
 (segment (start 105.41 69.85) (end 105.41 66.04) (width 1) (layer F.Cu) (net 7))
 (segment (start 116.84 71.12) (end 116.84 70.104) (width 0.254) (layer B.Cu) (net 7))
 (segment (start 116.84 70.104) (end 116.586 69.85) (width 0.254) (layer B.Cu) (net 7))
 (segment (start 116.586 69.85) (end 105.41 69.85) (width 0.254) (layer B.Cu) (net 7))
 (via (at 105.41 69.85) (size 0.6) (layers F.Cu B.Cu) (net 7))
 (segment (start 102.87 73.025) (end 102.87 73.66) (width 1) (layer F.Cu) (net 6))
 (segment (start 102.87 73.025) (end 102.87 69.088) (width 1) (layer F.Cu) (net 6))
 (segment (start 102.87 69.088) (end 102.87 66.04) (width 1) (layer F.Cu) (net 6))
 (segment (start 118.11 71.12) (end 118.11 70.104) (width 0.254) (layer B.Cu) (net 6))
 (segment (start 118.11 70.104) (end 117.094 69.088) (width 0.254) (layer B.Cu) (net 6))
 (segment (start 117.094 69.088) (end 102.87 69.088) (width 0.254) (layer B.Cu) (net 6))
 (via (at 102.87 69.088) (size 0.6) (layers F.Cu B.Cu) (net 6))
 (segment (start 100.33 73.66) (end 100.33 73.025) (width 1) (layer F.Cu) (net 5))
 (segment (start 100.33 80.518) (end 100.33 73.66) (width 0.254) (layer F.Cu) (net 5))
 (segment (start 100.33 73.025) (end 100.33 66.04) (width 1) (layer F.Cu) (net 5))
 (segment (start 129.54 88.9) (end 129.54 90.424) (width 0.254) (layer B.Cu) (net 5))
 (segment (start 129.54 90.424) (end 128.27 91.694) (width 0.254) (layer B.Cu) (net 5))
 (segment (start 128.27 91.694) (end 109.982 91.694) (width 0.254) (layer B.Cu) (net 5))
 (segment (start 109.982 91.694) (end 100.33 82.042) (width 0.254) (layer B.Cu) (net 5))
 (segment (start 100.33 82.042) (end 100.33 80.518) (width 0.254) (layer B.Cu) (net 5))
 (via (at 100.33 80.518) (size 0.6) (layers F.Cu B.Cu) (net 5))
 (segment (start 128.27 86.36) (end 128.27 93.98) (width 1) (layer F.Cu) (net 29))
 (segment (start 135.89 73.025) (end 135.89 73.66) (width 1) (layer F.Cu) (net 8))
 (segment (start 135.89 73.025) (end 135.89 66.04) (width 1) (layer F.Cu) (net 8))
 (segment (start 100.33 93.98) (end 100.33 86.36) (width 1) (layer F.Cu) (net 19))
 (segment (start 105.41 93.98) (end 105.41 86.36) (width 1) (layer F.Cu) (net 20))
 (segment (start 107.95 93.98) (end 107.95 86.36) (width 1) (layer F.Cu) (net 21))
 (segment (start 110.49 93.98) (end 110.49 86.36) (width 1) (layer F.Cu) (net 22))
 (segment (start 113.03 93.98) (end 113.03 86.36) (width 1) (layer F.Cu) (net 23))
 (segment (start 115.57 93.98) (end 115.57 86.36) (width 1) (layer F.Cu) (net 24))
 (segment (start 118.11 93.98) (end 118.11 86.36) (width 1) (layer F.Cu) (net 25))
 (segment (start 120.65 93.98) (end 120.65 86.36) (width 1) (layer F.Cu) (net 26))
 (segment (start 123.19 93.98) (end 123.19 86.36) (width 1) (layer F.Cu) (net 27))
 (segment (start 125.73 93.98) (end 125.73 86.36) (width 1) (layer F.Cu) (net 28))
 (segment (start 130.81 73.66) (end 130.81 66.04) (width 0.254) (layer F.Cu) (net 10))
 (segment (start 130.81 86.36) (end 130.81 73.66) (width 0.254) (layer F.Cu) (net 10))
 (segment (start 130.81 93.98) (end 130.81 86.36) (width 1) (layer F.Cu) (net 10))
 (segment (start 135.89 86.36) (end 135.89 93.98) (width 1) (layer F.Cu) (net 30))
 (segment (start 133.35 73.025) (end 133.35 73.66) (width 1) (layer F.Cu) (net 9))
 (segment (start 133.35 73.025) (end 133.35 66.04) (width 1) (layer F.Cu) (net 9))
 (segment (start 125.73 73.025) (end 125.73 73.66) (width 1) (layer F.Cu) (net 11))
 (segment (start 125.73 73.025) (end 125.73 66.04) (width 1) (layer F.Cu) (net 11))
 (segment (start 123.19 73.025) (end 123.19 73.66) (width 1) (layer F.Cu) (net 12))
 (segment (start 123.19 73.025) (end 123.19 66.04) (width 1) (layer F.Cu) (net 12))
 (segment (start 120.65 73.025) (end 120.65 73.66) (width 1) (layer F.Cu) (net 13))
 (segment (start 120.65 73.025) (end 120.65 66.04) (width 1) (layer F.Cu) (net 13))
 (segment (start 118.11 73.025) (end 118.11 73.66) (width 1) (layer F.Cu) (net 14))
 (segment (start 118.11 73.025) (end 118.11 66.04) (width 1) (layer F.Cu) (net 14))
 (segment (start 115.57 73.025) (end 115.57 73.66) (width 1) (layer F.Cu) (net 15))
 (segment (start 115.57 73.025) (end 115.57 66.04) (width 1) (layer F.Cu) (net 15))
 (segment (start 113.03 73.025) (end 113.03 73.66) (width 1) (layer F.Cu) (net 16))
 (segment (start 113.03 73.025) (end 113.03 66.04) (width 1) (layer F.Cu) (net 16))
 (segment (start 110.49 73.025) (end 110.49 73.66) (width 1) (layer F.Cu) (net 17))
 (segment (start 110.49 73.025) (end 110.49 66.04) (width 1) (layer F.Cu) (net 17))
 (segment (start 107.95 73.025) (end 107.95 73.66) (width 1) (layer F.Cu) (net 18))
 (segment (start 107.95 73.025) (end 107.95 66.04) (width 1) (layer F.Cu) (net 18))
 (segment (start 135.89 81.28) (end 142.24 81.28) (width 1) (layer B.Cu) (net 1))
 (segment (start 135.89 78.74) (end 137.668 78.74) (width 1) (layer B.Cu) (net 2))
 (segment (start 137.668 78.74) (end 140.208 76.2) (width 1) (layer B.Cu) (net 2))
 (segment (start 140.208 76.2) (end 142.24 76.2) (width 1) (layer B.Cu) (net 2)))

